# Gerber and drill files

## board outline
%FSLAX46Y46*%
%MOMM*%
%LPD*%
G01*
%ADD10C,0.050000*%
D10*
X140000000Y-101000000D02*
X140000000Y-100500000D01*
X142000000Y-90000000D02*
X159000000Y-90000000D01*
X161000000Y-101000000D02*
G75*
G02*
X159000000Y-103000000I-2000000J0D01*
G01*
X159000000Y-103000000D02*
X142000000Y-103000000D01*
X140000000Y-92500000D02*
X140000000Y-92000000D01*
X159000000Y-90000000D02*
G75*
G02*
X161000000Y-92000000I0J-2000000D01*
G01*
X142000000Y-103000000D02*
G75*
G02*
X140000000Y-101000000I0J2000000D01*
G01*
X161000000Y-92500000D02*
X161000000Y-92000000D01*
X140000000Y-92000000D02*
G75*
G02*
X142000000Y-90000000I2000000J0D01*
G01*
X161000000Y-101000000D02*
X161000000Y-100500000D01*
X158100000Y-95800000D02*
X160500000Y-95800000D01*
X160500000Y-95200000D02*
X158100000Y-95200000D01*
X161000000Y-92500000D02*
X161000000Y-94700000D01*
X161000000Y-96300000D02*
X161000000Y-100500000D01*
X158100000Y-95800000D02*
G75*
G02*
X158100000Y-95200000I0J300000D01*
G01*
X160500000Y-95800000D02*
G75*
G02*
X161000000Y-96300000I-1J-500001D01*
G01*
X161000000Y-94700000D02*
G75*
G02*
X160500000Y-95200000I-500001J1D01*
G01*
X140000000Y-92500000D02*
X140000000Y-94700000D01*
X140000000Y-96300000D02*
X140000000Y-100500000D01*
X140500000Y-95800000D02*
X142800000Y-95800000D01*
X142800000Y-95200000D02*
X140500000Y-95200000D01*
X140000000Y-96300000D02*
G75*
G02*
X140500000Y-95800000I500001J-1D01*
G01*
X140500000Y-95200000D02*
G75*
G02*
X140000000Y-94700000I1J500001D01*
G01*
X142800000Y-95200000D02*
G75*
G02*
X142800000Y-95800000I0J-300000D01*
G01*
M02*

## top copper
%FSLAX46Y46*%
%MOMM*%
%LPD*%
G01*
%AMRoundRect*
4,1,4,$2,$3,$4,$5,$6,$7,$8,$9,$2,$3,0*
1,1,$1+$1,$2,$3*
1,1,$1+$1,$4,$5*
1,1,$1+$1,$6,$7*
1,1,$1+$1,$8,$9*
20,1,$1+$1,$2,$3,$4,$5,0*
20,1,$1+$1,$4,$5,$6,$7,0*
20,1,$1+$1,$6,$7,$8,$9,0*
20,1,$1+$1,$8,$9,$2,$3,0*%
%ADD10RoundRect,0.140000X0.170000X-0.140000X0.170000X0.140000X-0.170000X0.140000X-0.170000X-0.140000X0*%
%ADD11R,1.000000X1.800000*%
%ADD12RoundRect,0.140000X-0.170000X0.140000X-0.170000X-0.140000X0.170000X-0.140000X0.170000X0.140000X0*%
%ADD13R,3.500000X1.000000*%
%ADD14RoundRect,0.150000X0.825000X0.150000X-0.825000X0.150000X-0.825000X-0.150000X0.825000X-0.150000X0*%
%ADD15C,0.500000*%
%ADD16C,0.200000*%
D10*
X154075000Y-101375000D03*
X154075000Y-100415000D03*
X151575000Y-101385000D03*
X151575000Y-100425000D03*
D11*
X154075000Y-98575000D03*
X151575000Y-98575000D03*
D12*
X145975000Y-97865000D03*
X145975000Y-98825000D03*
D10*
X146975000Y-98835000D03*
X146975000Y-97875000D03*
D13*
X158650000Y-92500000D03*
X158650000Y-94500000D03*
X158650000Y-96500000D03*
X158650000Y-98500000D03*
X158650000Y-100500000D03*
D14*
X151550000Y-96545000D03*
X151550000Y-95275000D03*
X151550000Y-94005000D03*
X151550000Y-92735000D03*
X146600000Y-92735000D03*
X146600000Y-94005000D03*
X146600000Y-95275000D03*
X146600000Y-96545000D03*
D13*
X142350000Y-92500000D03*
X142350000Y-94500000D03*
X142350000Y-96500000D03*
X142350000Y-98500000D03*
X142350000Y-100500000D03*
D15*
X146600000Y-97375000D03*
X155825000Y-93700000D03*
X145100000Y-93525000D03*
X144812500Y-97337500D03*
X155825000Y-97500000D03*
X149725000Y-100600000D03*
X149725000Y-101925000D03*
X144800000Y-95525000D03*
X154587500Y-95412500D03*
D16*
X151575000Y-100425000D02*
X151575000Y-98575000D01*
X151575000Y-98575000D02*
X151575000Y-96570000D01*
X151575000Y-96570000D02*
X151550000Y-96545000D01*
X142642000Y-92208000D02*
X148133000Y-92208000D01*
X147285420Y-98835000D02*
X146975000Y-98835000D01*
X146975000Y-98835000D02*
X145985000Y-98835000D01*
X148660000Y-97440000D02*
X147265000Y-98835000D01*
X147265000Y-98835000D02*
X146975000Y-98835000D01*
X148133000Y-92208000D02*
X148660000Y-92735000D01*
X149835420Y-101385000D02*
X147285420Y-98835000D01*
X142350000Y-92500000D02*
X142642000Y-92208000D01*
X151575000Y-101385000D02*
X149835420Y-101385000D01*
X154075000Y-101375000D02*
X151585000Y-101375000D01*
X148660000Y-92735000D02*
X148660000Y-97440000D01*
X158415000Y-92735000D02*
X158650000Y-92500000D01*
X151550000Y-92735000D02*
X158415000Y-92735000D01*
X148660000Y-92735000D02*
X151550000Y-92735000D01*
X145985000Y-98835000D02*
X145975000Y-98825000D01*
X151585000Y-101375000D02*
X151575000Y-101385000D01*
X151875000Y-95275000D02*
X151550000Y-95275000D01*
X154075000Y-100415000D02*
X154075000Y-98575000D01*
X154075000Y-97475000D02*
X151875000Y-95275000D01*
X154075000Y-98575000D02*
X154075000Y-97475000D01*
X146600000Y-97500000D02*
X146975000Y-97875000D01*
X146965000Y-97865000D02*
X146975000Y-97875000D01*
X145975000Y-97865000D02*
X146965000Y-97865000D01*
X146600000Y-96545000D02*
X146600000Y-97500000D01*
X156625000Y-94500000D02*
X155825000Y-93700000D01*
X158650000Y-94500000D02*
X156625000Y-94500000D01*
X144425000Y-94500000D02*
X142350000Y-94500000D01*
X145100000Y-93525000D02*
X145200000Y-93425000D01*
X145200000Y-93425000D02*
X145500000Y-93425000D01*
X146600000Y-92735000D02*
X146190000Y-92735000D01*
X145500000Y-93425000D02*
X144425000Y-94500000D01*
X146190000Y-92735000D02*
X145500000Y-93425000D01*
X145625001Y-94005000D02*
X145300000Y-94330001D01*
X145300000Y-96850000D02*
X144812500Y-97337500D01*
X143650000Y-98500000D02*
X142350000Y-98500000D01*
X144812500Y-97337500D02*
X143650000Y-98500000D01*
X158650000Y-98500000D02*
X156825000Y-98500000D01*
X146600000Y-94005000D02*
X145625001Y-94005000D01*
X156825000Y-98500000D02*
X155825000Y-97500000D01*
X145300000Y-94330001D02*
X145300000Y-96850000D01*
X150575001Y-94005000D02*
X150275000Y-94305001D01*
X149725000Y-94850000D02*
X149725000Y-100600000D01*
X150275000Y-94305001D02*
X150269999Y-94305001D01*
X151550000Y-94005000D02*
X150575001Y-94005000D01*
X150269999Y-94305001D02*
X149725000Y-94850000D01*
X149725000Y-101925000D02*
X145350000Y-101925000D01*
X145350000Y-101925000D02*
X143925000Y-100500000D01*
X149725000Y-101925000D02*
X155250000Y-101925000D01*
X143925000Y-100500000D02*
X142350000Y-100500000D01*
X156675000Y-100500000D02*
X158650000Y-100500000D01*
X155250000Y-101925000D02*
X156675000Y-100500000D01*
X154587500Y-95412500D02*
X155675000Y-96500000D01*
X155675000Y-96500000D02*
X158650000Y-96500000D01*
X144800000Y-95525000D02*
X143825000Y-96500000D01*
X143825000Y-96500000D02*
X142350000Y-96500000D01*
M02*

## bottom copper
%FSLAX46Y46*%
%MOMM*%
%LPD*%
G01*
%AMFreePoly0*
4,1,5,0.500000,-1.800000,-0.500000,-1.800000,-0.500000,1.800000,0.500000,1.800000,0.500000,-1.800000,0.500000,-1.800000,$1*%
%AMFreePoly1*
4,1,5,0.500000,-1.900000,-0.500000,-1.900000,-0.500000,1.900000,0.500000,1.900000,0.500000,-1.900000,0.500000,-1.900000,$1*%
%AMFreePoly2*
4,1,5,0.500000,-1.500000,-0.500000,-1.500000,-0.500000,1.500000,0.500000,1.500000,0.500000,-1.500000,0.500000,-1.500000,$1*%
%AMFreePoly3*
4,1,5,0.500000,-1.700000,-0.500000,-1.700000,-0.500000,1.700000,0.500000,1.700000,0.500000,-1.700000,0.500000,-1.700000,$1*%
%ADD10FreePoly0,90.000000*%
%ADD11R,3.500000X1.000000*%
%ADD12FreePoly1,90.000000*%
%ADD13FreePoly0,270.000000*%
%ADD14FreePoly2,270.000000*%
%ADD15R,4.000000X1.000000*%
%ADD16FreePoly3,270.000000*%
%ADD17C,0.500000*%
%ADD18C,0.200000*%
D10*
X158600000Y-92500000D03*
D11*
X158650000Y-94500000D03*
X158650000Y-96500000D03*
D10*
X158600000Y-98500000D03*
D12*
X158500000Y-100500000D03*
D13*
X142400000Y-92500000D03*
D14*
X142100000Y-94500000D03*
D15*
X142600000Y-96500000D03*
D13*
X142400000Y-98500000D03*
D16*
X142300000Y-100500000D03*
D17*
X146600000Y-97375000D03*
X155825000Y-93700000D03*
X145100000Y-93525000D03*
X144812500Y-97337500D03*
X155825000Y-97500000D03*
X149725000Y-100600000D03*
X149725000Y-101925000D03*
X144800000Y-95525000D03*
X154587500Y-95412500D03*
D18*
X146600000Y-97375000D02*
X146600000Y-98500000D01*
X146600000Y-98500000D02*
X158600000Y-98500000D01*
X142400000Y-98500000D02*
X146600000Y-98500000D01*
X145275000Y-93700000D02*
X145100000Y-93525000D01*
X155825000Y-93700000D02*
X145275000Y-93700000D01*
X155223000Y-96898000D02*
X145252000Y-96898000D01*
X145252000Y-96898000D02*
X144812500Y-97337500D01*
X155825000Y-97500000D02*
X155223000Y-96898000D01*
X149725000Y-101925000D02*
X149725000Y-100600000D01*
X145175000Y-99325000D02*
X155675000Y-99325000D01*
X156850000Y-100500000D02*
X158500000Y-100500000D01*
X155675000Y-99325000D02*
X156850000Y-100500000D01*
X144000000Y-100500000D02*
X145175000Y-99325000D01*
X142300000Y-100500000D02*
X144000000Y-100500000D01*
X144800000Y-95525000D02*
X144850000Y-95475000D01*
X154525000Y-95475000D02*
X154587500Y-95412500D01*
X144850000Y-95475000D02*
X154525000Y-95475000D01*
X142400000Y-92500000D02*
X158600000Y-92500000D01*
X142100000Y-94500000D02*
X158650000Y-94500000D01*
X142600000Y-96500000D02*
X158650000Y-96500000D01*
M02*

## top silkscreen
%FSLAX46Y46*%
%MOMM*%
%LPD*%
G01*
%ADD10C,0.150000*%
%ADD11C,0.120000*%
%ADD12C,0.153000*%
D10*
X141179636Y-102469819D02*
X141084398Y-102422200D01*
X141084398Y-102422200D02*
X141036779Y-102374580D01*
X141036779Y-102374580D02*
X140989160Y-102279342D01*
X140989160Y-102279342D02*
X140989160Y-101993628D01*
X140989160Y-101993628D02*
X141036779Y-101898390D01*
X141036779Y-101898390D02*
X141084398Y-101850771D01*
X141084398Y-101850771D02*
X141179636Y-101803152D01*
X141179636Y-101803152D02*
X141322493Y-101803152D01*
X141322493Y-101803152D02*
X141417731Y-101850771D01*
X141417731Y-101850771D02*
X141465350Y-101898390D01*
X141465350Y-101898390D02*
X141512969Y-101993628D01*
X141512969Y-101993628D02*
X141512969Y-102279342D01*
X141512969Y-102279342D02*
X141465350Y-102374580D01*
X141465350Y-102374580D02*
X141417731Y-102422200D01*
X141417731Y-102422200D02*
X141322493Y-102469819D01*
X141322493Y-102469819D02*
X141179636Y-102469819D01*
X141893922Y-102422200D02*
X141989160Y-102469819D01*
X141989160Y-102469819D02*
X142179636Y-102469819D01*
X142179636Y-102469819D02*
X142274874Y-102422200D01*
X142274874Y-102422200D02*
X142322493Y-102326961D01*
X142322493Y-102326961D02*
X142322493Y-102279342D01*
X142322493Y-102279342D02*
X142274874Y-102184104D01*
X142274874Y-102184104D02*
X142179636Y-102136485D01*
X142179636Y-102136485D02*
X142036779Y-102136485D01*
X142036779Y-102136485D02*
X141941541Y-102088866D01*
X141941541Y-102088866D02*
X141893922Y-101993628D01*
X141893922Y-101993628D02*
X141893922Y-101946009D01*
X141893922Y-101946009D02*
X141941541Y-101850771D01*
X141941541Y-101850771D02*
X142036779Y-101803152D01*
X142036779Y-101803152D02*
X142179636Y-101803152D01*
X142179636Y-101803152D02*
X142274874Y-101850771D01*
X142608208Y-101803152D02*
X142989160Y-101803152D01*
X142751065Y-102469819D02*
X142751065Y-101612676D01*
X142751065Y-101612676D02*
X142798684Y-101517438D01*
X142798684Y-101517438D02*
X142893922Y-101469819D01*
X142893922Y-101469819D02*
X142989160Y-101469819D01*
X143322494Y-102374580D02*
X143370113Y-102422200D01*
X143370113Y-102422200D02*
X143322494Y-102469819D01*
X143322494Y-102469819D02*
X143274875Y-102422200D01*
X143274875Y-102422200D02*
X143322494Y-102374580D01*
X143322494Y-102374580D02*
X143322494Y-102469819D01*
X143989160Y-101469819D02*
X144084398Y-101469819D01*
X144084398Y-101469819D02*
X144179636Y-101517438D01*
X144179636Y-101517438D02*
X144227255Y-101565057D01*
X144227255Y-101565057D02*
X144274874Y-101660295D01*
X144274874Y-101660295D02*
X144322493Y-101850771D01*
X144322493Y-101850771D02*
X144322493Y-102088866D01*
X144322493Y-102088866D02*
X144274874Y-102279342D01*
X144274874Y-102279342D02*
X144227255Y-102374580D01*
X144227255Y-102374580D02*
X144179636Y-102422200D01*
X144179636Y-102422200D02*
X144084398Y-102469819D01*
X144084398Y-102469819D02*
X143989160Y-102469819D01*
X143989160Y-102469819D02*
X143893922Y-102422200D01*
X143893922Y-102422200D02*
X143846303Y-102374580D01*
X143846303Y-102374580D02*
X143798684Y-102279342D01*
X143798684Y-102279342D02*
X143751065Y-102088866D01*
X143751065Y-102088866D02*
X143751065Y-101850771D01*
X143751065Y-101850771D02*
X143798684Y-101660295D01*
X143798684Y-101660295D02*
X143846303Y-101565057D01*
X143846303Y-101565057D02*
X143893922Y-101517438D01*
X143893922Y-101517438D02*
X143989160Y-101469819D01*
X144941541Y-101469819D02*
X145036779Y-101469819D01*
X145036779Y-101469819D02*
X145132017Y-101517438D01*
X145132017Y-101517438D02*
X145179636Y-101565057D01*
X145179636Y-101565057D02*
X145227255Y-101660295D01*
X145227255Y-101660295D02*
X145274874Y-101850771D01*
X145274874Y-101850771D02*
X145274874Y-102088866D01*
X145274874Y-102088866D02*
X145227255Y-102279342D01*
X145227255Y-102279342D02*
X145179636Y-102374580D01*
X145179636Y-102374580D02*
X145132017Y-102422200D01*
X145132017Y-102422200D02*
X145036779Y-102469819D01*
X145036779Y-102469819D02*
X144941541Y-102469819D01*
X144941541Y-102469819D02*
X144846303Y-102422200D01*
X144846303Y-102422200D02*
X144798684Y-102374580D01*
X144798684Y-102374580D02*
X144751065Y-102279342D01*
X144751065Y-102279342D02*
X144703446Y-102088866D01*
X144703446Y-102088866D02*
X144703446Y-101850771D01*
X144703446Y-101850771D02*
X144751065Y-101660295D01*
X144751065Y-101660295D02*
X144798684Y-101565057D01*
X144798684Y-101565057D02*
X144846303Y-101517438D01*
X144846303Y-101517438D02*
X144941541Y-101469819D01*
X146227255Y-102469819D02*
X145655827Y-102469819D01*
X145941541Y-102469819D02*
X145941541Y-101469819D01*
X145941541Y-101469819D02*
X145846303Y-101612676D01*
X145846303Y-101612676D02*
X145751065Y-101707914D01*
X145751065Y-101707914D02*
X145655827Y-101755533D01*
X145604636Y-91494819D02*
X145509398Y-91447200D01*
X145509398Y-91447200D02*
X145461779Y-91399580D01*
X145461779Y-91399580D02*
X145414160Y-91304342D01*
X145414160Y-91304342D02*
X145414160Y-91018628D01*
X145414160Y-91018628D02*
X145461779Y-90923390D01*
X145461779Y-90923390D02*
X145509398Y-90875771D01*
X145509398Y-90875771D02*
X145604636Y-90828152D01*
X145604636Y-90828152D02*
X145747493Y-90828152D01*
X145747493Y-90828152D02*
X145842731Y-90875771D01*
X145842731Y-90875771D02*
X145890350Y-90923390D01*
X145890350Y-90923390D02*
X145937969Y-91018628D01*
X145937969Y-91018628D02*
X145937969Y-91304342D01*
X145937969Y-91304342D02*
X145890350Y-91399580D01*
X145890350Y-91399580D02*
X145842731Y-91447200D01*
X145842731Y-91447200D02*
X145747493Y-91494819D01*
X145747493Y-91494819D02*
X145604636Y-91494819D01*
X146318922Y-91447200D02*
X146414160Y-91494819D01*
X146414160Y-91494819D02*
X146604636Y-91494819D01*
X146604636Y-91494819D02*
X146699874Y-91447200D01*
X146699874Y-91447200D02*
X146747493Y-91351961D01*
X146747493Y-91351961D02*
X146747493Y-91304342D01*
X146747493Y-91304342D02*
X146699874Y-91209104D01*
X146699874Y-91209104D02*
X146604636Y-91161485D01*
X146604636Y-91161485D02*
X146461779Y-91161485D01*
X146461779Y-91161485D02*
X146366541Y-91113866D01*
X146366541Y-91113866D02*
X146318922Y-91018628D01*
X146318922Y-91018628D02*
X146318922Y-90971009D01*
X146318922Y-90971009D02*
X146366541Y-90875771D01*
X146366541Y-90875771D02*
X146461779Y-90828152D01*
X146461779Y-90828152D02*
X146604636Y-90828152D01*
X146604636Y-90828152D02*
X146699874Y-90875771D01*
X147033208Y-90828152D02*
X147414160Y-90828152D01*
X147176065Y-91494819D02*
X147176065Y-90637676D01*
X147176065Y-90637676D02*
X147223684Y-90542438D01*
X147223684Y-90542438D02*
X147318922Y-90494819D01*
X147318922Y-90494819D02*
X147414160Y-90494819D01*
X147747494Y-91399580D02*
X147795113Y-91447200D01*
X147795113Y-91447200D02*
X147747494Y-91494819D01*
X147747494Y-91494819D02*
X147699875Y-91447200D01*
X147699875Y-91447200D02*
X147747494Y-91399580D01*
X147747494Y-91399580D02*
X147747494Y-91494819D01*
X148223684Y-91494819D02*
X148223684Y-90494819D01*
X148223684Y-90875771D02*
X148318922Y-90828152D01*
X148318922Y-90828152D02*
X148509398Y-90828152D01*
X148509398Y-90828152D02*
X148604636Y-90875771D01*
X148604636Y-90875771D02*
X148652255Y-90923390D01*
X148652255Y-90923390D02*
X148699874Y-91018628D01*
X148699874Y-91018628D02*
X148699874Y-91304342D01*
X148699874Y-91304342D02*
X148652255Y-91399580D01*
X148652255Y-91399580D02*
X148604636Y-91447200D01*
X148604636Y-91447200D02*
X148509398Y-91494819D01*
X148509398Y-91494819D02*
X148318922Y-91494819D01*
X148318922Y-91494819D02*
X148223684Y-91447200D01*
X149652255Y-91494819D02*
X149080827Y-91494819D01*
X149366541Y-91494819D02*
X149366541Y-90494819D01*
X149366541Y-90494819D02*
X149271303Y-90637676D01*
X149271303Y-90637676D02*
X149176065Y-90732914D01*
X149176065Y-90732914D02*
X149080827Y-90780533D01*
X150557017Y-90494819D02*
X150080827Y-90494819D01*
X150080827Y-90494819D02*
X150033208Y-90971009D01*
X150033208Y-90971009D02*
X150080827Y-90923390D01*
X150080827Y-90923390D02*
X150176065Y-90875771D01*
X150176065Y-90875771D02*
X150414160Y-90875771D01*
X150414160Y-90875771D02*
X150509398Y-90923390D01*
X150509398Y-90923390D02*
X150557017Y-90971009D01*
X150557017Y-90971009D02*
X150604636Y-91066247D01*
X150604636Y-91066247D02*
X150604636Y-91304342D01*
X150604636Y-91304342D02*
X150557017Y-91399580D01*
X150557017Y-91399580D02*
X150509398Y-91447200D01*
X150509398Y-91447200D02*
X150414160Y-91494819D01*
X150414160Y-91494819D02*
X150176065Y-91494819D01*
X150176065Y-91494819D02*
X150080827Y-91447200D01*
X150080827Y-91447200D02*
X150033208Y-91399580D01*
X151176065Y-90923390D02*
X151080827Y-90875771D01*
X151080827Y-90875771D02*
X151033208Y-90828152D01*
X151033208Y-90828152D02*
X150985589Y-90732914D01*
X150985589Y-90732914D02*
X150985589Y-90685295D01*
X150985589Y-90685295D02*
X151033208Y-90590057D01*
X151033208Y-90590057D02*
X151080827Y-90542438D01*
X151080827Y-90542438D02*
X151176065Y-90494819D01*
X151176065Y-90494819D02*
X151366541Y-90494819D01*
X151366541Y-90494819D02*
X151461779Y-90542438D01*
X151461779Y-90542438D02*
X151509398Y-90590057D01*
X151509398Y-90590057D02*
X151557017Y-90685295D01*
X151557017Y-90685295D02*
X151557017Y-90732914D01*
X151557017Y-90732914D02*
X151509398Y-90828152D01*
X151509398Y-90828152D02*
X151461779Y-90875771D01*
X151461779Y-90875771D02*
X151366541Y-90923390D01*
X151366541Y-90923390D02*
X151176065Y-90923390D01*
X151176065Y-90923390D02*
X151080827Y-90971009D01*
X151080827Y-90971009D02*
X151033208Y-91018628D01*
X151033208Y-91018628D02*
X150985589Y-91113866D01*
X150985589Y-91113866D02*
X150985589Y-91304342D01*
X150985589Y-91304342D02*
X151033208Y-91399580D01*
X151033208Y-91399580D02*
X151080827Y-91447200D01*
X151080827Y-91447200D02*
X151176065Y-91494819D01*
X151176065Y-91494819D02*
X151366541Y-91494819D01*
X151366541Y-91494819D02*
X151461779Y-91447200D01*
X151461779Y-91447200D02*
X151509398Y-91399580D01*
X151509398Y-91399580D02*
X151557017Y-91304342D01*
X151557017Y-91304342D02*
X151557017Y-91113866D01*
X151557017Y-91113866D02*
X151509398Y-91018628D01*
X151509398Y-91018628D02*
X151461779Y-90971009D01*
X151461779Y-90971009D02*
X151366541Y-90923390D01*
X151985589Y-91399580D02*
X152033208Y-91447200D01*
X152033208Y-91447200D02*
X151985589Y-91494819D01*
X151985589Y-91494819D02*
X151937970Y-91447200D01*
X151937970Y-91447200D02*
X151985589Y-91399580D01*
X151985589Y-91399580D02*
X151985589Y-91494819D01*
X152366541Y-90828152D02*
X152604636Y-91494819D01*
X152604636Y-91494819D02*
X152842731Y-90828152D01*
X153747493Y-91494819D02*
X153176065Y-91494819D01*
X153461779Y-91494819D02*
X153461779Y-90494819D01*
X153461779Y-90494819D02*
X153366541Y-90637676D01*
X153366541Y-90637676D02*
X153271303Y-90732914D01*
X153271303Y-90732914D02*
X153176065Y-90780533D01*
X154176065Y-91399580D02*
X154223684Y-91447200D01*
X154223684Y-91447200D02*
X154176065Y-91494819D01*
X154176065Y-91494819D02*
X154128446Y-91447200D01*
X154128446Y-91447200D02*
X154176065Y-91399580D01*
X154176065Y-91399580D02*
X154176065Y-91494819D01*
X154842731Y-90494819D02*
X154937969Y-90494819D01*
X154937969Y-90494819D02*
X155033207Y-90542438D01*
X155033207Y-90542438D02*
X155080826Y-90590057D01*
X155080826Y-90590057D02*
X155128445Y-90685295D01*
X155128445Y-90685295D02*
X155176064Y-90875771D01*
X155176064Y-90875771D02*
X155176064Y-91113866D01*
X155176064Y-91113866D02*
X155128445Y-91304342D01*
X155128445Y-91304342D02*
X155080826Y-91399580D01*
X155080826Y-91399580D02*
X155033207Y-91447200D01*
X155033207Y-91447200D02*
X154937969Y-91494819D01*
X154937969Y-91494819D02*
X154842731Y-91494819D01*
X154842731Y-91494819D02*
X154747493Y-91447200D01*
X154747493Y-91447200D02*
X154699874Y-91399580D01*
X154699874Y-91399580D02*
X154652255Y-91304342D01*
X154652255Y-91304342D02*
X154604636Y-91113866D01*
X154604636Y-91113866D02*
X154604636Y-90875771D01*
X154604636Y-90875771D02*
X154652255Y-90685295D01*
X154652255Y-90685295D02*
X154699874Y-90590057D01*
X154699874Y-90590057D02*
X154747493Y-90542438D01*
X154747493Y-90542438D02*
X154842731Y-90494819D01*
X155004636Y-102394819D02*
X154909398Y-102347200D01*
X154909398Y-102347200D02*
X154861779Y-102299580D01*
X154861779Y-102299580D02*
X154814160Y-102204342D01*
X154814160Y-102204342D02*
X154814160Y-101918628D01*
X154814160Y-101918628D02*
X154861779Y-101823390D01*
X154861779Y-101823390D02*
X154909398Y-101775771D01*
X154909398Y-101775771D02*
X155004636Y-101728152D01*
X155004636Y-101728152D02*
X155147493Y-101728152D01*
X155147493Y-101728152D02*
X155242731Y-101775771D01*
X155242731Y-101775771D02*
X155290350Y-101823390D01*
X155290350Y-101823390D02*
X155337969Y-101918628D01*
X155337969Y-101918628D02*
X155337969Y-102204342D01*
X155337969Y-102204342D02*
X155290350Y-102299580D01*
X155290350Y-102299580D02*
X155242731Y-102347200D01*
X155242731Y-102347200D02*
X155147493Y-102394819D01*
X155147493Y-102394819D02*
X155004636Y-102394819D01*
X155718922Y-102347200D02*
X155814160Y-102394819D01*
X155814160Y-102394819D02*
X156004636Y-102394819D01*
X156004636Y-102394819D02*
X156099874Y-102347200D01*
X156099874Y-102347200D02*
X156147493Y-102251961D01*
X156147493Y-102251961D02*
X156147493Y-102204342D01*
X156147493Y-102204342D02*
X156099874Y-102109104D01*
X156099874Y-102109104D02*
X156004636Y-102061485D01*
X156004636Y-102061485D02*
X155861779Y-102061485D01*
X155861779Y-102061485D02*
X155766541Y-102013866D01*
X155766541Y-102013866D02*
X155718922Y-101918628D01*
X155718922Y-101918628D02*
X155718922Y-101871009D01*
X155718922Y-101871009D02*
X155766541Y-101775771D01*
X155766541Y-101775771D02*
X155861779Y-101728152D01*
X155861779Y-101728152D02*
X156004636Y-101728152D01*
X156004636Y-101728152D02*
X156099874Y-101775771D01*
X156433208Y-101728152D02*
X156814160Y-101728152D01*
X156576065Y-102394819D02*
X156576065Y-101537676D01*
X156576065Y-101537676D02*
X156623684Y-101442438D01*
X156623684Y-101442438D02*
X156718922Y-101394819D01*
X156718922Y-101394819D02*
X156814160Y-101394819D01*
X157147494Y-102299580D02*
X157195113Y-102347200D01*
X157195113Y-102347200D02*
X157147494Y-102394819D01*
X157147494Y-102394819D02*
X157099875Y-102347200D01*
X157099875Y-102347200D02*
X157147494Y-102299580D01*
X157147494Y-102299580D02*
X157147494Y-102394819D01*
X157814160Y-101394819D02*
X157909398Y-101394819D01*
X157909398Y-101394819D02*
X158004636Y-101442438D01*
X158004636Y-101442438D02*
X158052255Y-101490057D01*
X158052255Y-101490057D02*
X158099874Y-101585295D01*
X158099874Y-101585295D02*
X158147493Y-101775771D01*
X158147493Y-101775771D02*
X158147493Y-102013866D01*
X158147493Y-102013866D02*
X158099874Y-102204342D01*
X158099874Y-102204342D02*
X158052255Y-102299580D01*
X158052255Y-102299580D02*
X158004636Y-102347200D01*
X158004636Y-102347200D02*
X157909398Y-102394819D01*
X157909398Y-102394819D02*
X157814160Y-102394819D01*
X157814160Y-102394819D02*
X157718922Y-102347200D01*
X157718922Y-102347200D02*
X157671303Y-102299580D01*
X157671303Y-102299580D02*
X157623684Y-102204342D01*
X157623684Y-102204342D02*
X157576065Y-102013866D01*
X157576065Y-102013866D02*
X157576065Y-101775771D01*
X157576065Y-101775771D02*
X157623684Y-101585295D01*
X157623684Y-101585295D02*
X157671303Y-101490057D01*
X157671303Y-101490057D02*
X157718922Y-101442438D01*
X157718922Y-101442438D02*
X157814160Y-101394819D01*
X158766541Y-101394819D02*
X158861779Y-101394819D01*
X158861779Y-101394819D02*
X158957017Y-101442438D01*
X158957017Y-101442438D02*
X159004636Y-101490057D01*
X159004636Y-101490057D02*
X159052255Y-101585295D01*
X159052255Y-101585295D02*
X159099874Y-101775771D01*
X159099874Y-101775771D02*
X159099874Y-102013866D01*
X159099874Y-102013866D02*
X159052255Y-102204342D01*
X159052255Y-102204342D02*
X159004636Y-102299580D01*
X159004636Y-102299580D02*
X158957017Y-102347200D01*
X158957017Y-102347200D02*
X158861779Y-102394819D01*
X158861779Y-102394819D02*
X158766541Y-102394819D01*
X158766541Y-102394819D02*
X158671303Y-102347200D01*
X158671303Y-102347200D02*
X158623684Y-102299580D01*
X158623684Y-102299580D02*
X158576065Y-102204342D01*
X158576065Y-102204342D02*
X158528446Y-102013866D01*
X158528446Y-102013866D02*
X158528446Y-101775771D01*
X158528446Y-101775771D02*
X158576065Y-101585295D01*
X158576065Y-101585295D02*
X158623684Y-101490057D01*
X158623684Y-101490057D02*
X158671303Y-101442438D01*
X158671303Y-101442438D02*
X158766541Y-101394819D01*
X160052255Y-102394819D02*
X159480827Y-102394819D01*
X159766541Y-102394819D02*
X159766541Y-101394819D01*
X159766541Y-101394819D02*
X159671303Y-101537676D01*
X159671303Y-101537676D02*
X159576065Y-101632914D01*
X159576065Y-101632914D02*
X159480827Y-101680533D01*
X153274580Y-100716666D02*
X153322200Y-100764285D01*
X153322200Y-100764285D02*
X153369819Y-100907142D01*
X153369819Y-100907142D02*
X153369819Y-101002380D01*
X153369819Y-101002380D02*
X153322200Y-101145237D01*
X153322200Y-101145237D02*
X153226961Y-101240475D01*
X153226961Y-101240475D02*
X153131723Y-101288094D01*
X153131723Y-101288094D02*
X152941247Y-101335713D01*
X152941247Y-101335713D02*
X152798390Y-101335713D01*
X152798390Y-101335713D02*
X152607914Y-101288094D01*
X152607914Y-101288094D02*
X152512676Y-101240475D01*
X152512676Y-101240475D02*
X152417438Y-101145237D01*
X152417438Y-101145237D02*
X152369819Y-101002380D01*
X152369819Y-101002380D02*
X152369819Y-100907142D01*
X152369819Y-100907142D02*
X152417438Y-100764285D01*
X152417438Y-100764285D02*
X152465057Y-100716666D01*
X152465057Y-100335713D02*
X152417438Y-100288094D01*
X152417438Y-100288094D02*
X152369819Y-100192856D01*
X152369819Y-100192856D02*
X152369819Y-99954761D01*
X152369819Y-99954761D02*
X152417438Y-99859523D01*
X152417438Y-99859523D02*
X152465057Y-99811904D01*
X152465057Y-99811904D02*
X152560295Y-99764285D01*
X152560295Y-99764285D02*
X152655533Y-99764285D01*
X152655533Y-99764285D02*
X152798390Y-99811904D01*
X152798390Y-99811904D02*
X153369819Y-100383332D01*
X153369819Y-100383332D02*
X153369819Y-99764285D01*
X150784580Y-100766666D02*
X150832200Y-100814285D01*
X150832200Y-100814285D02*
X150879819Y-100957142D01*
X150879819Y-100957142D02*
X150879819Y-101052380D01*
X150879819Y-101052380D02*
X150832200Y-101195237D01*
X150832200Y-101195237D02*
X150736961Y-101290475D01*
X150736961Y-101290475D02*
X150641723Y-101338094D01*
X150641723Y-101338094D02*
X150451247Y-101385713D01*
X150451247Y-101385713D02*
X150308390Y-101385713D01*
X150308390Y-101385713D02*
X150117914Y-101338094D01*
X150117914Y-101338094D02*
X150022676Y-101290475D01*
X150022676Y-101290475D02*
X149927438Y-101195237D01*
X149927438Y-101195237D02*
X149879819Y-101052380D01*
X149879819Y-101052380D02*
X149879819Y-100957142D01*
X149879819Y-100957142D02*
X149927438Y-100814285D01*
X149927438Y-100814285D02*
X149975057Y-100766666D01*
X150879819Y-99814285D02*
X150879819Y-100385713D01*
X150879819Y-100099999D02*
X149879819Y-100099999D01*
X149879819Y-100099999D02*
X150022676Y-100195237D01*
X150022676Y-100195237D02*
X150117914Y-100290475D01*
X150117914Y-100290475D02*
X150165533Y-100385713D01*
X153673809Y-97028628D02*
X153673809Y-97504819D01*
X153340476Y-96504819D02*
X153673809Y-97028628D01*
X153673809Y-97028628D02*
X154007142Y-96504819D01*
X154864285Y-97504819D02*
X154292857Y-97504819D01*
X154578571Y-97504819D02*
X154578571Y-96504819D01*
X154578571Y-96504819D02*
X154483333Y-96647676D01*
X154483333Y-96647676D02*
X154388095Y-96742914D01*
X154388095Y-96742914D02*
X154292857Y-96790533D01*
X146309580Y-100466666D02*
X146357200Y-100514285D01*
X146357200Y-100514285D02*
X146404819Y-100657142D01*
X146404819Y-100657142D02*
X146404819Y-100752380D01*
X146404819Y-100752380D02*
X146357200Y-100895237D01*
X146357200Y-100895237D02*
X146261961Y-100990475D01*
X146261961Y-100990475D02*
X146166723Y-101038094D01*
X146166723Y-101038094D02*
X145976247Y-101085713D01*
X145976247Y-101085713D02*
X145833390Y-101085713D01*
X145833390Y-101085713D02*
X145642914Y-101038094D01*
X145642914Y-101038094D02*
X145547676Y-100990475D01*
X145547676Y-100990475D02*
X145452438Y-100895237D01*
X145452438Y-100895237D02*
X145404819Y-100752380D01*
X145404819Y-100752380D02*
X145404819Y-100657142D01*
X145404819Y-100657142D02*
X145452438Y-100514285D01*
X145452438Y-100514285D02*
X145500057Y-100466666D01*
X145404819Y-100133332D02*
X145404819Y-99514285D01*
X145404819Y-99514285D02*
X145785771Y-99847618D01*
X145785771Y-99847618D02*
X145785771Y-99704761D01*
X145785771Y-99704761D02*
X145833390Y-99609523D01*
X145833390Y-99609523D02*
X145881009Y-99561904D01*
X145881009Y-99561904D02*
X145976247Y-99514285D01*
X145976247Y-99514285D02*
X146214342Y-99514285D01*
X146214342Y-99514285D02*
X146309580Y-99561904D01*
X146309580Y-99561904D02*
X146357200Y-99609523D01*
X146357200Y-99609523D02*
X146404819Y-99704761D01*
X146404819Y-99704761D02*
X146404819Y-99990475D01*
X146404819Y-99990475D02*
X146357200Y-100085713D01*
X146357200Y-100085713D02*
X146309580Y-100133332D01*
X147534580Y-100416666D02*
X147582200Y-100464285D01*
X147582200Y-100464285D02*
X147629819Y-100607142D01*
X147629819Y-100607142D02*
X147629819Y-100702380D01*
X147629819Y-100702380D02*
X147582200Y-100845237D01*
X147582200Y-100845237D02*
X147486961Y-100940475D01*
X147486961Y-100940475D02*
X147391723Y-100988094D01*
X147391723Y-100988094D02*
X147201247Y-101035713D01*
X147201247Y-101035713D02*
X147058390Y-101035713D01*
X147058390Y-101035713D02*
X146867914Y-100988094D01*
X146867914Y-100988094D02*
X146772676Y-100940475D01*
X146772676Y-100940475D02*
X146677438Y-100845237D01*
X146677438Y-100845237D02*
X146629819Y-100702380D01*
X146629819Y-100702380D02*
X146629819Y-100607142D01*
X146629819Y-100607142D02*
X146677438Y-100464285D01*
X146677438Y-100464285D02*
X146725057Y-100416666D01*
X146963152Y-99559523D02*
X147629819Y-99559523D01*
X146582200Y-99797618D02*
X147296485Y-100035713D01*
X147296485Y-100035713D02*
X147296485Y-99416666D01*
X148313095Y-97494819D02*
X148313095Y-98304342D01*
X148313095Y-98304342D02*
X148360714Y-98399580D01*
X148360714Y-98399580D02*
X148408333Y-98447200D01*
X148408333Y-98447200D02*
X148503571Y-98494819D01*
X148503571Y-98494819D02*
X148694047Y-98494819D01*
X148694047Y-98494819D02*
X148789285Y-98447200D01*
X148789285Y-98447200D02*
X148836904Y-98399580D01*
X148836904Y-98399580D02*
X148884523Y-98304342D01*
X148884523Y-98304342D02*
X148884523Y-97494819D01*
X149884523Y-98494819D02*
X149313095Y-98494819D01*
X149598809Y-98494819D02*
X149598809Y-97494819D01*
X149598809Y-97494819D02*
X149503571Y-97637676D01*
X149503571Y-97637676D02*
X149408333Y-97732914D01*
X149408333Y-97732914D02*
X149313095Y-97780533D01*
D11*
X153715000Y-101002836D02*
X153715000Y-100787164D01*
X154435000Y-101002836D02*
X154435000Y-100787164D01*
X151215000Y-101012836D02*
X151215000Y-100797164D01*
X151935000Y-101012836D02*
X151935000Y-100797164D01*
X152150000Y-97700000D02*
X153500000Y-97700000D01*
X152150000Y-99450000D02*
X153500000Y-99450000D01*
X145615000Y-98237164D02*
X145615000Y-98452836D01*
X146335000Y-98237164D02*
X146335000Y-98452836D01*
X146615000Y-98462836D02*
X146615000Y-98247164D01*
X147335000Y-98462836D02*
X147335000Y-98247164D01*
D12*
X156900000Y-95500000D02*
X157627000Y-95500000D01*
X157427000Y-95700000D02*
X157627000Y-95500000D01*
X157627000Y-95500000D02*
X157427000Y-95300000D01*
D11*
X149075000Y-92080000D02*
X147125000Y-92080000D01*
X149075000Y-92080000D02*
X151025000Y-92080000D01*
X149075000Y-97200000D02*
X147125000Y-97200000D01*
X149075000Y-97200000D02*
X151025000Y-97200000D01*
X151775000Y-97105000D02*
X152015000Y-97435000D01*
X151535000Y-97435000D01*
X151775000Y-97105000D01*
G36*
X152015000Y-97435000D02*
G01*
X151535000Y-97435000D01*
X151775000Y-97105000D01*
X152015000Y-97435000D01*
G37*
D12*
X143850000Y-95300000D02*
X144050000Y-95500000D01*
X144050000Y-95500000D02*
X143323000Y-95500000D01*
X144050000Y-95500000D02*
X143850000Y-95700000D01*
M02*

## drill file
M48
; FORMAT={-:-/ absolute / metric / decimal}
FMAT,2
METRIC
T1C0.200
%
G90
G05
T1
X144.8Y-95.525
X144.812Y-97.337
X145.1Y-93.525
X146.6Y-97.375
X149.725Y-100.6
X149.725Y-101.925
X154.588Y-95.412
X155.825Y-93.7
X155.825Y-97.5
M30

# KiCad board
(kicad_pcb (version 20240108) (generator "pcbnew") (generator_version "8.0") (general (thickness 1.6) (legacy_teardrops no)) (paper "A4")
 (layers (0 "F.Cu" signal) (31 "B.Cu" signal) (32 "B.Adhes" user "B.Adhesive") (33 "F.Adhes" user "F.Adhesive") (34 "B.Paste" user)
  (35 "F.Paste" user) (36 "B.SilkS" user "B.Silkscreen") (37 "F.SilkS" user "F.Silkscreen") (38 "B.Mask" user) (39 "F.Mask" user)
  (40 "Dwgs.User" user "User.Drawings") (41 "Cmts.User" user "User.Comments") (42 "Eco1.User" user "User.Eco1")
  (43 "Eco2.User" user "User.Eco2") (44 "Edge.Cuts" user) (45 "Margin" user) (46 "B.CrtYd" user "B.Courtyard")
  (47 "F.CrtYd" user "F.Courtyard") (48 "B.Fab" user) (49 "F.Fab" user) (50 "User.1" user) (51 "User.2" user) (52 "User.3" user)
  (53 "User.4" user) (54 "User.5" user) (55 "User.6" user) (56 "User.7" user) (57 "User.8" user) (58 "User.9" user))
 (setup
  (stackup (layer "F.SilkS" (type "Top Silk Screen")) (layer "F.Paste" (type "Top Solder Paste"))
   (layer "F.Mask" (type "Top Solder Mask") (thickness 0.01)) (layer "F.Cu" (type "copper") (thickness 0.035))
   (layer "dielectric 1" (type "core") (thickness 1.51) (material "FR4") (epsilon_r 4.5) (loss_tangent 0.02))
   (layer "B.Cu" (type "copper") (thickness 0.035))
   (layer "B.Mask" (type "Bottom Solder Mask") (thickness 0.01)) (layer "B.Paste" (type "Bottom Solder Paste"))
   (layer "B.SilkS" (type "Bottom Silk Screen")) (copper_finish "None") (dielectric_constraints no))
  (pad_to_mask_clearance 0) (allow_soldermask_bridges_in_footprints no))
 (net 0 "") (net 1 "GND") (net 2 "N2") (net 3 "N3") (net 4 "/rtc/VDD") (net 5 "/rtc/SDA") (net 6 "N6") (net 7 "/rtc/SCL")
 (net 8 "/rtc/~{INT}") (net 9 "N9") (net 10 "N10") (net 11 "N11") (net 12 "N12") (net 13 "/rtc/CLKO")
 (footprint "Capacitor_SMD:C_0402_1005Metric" (layer "F.Cu") (at 154.075 100.895 90)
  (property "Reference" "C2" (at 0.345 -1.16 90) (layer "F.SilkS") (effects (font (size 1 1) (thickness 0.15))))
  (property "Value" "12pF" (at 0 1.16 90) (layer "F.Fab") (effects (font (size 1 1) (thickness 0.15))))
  (fp_line (start -0.107836 -0.36) (end 0.107836 -0.36) (stroke (width 0.12) (type solid)) (layer "F.SilkS"))
  (fp_line (start -0.107836 0.36) (end 0.107836 0.36) (stroke (width 0.12) (type solid)) (layer "F.SilkS"))
  (pad "1" smd roundrect (at -0.48 0 90) (size 0.56 0.62) (layers "F.Cu" "F.Paste" "F.Mask") (roundrect_rratio 0.25) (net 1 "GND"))
  (pad "2" smd roundrect (at 0.48 0 90) (size 0.56 0.62) (layers "F.Cu" "F.Paste" "F.Mask") (roundrect_rratio 0.25) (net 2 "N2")))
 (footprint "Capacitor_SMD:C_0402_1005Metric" (layer "F.Cu") (at 151.575 100.905 90)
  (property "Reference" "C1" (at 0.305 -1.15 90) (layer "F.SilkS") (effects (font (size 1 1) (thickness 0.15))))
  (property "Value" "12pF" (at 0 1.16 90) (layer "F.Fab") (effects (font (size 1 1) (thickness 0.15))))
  (fp_line (start -0.107836 -0.36) (end 0.107836 -0.36) (stroke (width 0.12) (type solid)) (layer "F.SilkS"))
  (fp_line (start -0.107836 0.36) (end 0.107836 0.36) (stroke (width 0.12) (type solid)) (layer "F.SilkS"))
  (pad "1" smd roundrect (at -0.48 0 90) (size 0.56 0.62) (layers "F.Cu" "F.Paste" "F.Mask") (roundrect_rratio 0.25) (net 1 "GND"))
  (pad "2" smd roundrect (at 0.48 0 90) (size 0.56 0.62) (layers "F.Cu" "F.Paste" "F.Mask") (roundrect_rratio 0.25) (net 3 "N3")))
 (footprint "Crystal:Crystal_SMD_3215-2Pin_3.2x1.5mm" (layer "F.Cu") (at 152.825 98.575)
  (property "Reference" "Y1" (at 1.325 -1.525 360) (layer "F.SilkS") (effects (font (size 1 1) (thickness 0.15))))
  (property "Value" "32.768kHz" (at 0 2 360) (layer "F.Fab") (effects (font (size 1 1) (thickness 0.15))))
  (fp_line (start -0.675 -0.875) (end 0.675 -0.875) (stroke (width 0.12) (type solid)) (layer "F.SilkS"))
  (fp_line (start -0.675 0.875) (end 0.675 0.875) (stroke (width 0.12) (type solid)) (layer "F.SilkS"))
  (pad "1" smd rect (at 1.25 0) (size 1 1.8) (layers "F.Cu" "F.Paste" "F.Mask") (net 2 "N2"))
  (pad "2" smd rect (at -1.25 0) (size 1 1.8) (layers "F.Cu" "F.Paste" "F.Mask") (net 3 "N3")))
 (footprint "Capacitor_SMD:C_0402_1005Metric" (layer "F.Cu") (at 145.975 98.345 -90)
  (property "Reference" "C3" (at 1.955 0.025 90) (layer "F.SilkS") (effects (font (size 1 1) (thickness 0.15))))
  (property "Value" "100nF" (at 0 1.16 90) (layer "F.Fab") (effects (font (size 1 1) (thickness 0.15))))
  (fp_line (start -0.107836 0.36) (end 0.107836 0.36) (stroke (width 0.12) (type solid)) (layer "F.SilkS"))
  (fp_line (start -0.107836 -0.36) (end 0.107836 -0.36) (stroke (width 0.12) (type solid)) (layer "F.SilkS"))
  (pad "1" smd roundrect (at -0.48 0 270) (size 0.56 0.62) (layers "F.Cu" "F.Paste" "F.Mask") (roundrect_rratio 0.25) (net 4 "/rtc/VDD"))
  (pad "2" smd roundrect (at 0.48 0 270) (size 0.56 0.62) (layers "F.Cu" "F.Paste" "F.Mask") (roundrect_rratio 0.25) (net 1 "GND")))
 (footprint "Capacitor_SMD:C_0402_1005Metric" (layer "F.Cu") (at 146.975 98.355 90)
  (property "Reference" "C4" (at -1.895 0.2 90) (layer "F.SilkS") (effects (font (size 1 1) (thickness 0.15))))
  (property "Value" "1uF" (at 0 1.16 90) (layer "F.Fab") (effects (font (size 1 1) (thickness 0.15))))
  (fp_line (start -0.107836 -0.36) (end 0.107836 -0.36) (stroke (width 0.12) (type solid)) (layer "F.SilkS"))
  (fp_line (start -0.107836 0.36) (end 0.107836 0.36) (stroke (width 0.12) (type solid)) (layer "F.SilkS"))
  (pad "1" smd roundrect (at -0.48 0 90) (size 0.56 0.62) (layers "F.Cu" "F.Paste" "F.Mask") (roundrect_rratio 0.25) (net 1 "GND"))
  (pad "2" smd roundrect (at 0.48 0 90) (size 0.56 0.62) (layers "F.Cu" "F.Paste" "F.Mask") (roundrect_rratio 0.25) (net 4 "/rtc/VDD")))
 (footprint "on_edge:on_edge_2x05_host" (layer "F.Cu") (at 161 96.5 -90)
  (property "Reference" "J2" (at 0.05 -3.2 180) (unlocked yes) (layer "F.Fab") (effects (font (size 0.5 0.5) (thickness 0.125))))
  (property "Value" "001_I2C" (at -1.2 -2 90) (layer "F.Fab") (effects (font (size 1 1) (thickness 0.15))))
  (fp_line (start -1 4.1) (end -1 3.373) (stroke (width 0.153) (type solid)) (layer "F.SilkS"))
  (fp_line (start -0.8 3.573) (end -1 3.373) (stroke (width 0.153) (type solid)) (layer "F.SilkS"))
  (fp_line (start -1 3.373) (end -1.2 3.573) (stroke (width 0.153) (type solid)) (layer "F.SilkS"))
  (fp_line (start -0.7 2.9) (end -0.7 0.5) (stroke (width 0.05) (type solid)) (layer "Edge.Cuts"))
  (fp_line (start -1.3 0.5) (end -1.3 2.9) (stroke (width 0.05) (type solid)) (layer "Edge.Cuts"))
  (fp_line (start -4 0) (end -1.8 0) (stroke (width 0.05) (type solid)) (layer "Edge.Cuts"))
  (fp_line (start -0.2 0) (end 4 0) (stroke (width 0.05) (type solid)) (layer "Edge.Cuts"))
  (fp_arc (start -0.7 2.9) (mid -1 3.2) (end -1.3 2.9) (stroke (width 0.05) (type solid)) (layer "Edge.Cuts"))
  (fp_arc (start -0.7 0.5) (mid -0.553553 0.146447) (end -0.2 0) (stroke (width 0.05) (type solid)) (layer "Edge.Cuts"))
  (fp_arc (start -1.8 0) (mid -1.446447 0.146447) (end -1.3 0.5) (stroke (width 0.05) (type solid)) (layer "Edge.Cuts"))
  (pad "1" smd rect (at -4 2.35 270) (size 1 3.5) (layers "F.Cu" "F.Mask") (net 1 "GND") (zone_connect 0))
  (pad "2" smd rect (at -2 2.35 270) (size 1 3.5) (layers "F.Cu" "F.Mask") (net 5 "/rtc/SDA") (zone_connect 0))
  (pad "3" smd rect (at 0 2.35 270) (size 1 3.5) (layers "F.Cu" "F.Mask") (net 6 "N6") (zone_connect 0))
  (pad "4" smd rect (at 2 2.35 270) (size 1 3.5) (layers "F.Cu" "F.Mask") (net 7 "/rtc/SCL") (zone_connect 0))
  (pad "5" smd rect (at 4 2.35 270) (size 1 3.5) (layers "F.Cu" "F.Mask") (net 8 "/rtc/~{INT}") (zone_connect 0))
  (pad "6" smd custom (at -4 2.4 90) (size 1 3.6) (layers "B.Cu" "B.Mask") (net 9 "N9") (zone_connect 0)
   (options (clearance outline) (anchor rect)) (primitives))
  (pad "7" smd rect (at -2 2.35 90) (size 1 3.5) (layers "B.Cu" "B.Mask") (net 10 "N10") (zone_connect 0))
  (pad "8" smd rect (at 0 2.35 90) (size 1 3.5) (layers "B.Cu" "B.Mask") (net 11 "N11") (zone_connect 0))
  (pad "9" smd custom (at 2 2.4 90) (size 1 3.6) (layers "B.Cu" "B.Mask") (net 4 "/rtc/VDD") (zone_connect 0)
   (options (clearance outline) (anchor rect)) (primitives))
  (pad "10" smd custom (at 4 2.5 90) (size 1 3.8) (layers "B.Cu" "B.Mask") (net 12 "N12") (zone_connect 0)
   (options (clearance outline) (anchor rect)) (primitives))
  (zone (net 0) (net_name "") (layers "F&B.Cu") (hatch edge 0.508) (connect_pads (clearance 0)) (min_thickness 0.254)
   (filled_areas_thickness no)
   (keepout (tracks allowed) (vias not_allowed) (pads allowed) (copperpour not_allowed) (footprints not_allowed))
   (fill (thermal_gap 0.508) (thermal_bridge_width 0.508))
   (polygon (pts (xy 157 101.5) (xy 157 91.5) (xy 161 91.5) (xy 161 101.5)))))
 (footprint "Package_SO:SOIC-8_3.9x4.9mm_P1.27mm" (layer "F.Cu") (at 149.075 94.64 180)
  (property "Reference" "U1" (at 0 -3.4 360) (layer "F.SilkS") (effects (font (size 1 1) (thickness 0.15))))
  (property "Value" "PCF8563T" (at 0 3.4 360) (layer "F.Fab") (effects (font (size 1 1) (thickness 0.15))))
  (fp_line (start 0 2.56) (end 1.95 2.56) (stroke (width 0.12) (type solid)) (layer "F.SilkS"))
  (fp_line (start 0 2.56) (end -1.95 2.56) (stroke (width 0.12) (type solid)) (layer "F.SilkS"))
  (fp_line (start 0 -2.56) (end 1.95 -2.56) (stroke (width 0.12) (type solid)) (layer "F.SilkS"))
  (fp_line (start 0 -2.56) (end -1.95 -2.56) (stroke (width 0.12) (type solid)) (layer "F.SilkS"))
  (fp_poly
   (pts (xy -2.7 -2.465) (xy -2.94 -2.795) (xy -2.46 -2.795) (xy -2.7 -2.465)) (stroke (width 0.12) (type solid)) (fill solid)
   (layer "F.SilkS"))
  (pad "1" smd roundrect (at -2.475 -1.905 180) (size 1.95 0.6) (layers "F.Cu" "F.Paste" "F.Mask") (roundrect_rratio 0.25) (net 3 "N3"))
  (pad "2" smd roundrect (at -2.475 -0.635 180) (size 1.95 0.6) (layers "F.Cu" "F.Paste" "F.Mask") (roundrect_rratio 0.25) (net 2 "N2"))
  (pad "3" smd roundrect (at -2.475 0.635 180) (size 1.95 0.6) (layers "F.Cu" "F.Paste" "F.Mask") (roundrect_rratio 0.25)
   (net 8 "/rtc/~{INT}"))
  (pad "4" smd roundrect (at -2.475 1.905 180) (size 1.95 0.6) (layers "F.Cu" "F.Paste" "F.Mask") (roundrect_rratio 0.25) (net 1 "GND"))
  (pad "5" smd roundrect (at 2.475 1.905 180) (size 1.95 0.6) (layers "F.Cu" "F.Paste" "F.Mask") (roundrect_rratio 0.25) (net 5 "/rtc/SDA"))
  (pad "6" smd roundrect (at 2.475 0.635 180) (size 1.95 0.6) (layers "F.Cu" "F.Paste" "F.Mask") (roundrect_rratio 0.25) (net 7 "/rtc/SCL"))
  (pad "7" smd roundrect (at 2.475 -0.635 180) (size 1.95 0.6) (layers "F.Cu" "F.Paste" "F.Mask") (roundrect_rratio 0.25)
   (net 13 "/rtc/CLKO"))
  (pad "8" smd roundrect (at 2.475 -1.905 180) (size 1.95 0.6) (layers "F.Cu" "F.Paste" "F.Mask") (roundrect_rratio 0.25) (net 4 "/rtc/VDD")))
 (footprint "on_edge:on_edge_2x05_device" (layer "F.Cu") (at 140 96.5 -90)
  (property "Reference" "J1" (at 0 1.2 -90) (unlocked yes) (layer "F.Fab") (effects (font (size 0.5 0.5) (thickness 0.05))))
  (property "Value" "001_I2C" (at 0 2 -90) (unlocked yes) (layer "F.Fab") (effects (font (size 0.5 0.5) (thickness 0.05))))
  (fp_line (start -1.2 -3.85) (end -1 -4.05) (stroke (width 0.153) (type solid)) (layer "F.SilkS"))
  (fp_line (start -1 -4.05) (end -1 -3.323) (stroke (width 0.153) (type solid)) (layer "F.SilkS"))
  (fp_line (start -1 -4.05) (end -0.8 -3.85) (stroke (width 0.153) (type solid)) (layer "F.SilkS"))
  (fp_line (start -4 0) (end -1.8 0) (stroke (width 0.05) (type solid)) (layer "Edge.Cuts"))
  (fp_line (start -0.2 0) (end 4 0) (stroke (width 0.05) (type solid)) (layer "Edge.Cuts"))
  (fp_line (start -0.7 -0.5) (end -0.7 -2.8) (stroke (width 0.05) (type solid)) (layer "Edge.Cuts"))
  (fp_line (start -1.3 -2.8) (end -1.3 -0.5) (stroke (width 0.05) (type solid)) (layer "Edge.Cuts"))
  (fp_arc (start -0.2 0) (mid -0.553553 -0.146447) (end -0.7 -0.5) (stroke (width 0.05) (type solid)) (layer "Edge.Cuts"))
  (fp_arc (start -1.3 -0.5) (mid -1.446447 -0.146447) (end -1.8 0) (stroke (width 0.05) (type solid)) (layer "Edge.Cuts"))
  (fp_arc (start -1.3 -2.8) (mid -1 -3.1) (end -0.7 -2.8) (stroke (width 0.05) (type solid)) (layer "Edge.Cuts"))
  (pad "1" smd rect (at -4 -2.35 90) (size 1 3.5) (layers "F.Cu" "F.Mask") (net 1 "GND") (zone_connect 0))
  (pad "2" smd rect (at -2 -2.35 270) (size 1 3.5) (layers "F.Cu" "F.Mask") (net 5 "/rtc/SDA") (zone_connect 0))
  (pad "3" smd rect (at 0 -2.35 270) (size 1 3.5) (layers "F.Cu" "F.Mask") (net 6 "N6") (zone_connect 0))
  (pad "4" smd rect (at 2 -2.35 90) (size 1 3.5) (layers "F.Cu" "F.Mask") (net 7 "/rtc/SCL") (zone_connect 0))
  (pad "5" smd rect (at 4 -2.35 90) (size 1 3.5) (layers "F.Cu" "F.Mask") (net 8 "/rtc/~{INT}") (zone_connect 0))
  (pad "6" smd custom (at -4 -2.4 270) (size 1 3.6) (layers "B.Cu" "B.Mask") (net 9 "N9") (zone_connect 0)
   (options (clearance outline) (anchor rect)) (primitives))
  (pad "7" smd custom (at -2 -2.1 270) (size 1 3) (layers "B.Cu" "B.Mask") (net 10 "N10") (zone_connect 0)
   (options (clearance outline) (anchor rect)) (primitives))
  (pad "8" smd rect (at 0 -2.6 270) (size 1 4) (layers "B.Cu" "B.Mask") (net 11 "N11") (zone_connect 0))
  (pad "9" smd custom (at 2 -2.4 270) (size 1 3.6) (layers "B.Cu" "B.Mask") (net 4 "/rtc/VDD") (zone_connect 0)
   (options (clearance outline) (anchor rect)) (primitives))
  (pad "10" smd custom (at 4 -2.3 270) (size 1 3.4) (layers "B.Cu" "B.Mask") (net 12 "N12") (zone_connect 0)
   (options (clearance outline) (anchor rect)) (primitives))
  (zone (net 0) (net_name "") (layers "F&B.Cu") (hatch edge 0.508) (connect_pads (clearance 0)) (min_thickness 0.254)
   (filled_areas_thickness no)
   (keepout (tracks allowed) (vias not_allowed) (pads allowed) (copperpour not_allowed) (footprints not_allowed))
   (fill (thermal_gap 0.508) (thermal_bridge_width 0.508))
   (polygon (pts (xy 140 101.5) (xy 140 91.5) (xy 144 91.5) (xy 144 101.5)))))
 (gr_line (start 140 101) (end 140 100.5) (stroke (width 0.05) (type solid)) (layer "Edge.Cuts"))
 (gr_line (start 142 90) (end 159 90) (stroke (width 0.05) (type solid)) (layer "Edge.Cuts"))
 (gr_arc (start 161 101) (mid 160.414214 102.414214) (end 159 103) (stroke (width 0.05) (type solid)) (layer "Edge.Cuts"))
 (gr_line (start 159 103) (end 142 103) (stroke (width 0.05) (type solid)) (layer "Edge.Cuts"))
 (gr_line (start 140 92.5) (end 140 92) (stroke (width 0.05) (type solid)) (layer "Edge.Cuts"))
 (gr_arc (start 159 90) (mid 160.414214 90.585786) (end 161 92) (stroke (width 0.05) (type solid)) (layer "Edge.Cuts"))
 (gr_arc (start 142 103) (mid 140.585786 102.414214) (end 140 101) (stroke (width 0.05) (type solid)) (layer "Edge.Cuts"))
 (gr_line (start 161 92.5) (end 161 92) (stroke (width 0.05) (type solid)) (layer "Edge.Cuts"))
 (gr_arc (start 140 92) (mid 140.585786 90.585786) (end 142 90) (stroke (width 0.05) (type solid)) (layer "Edge.Cuts"))
 (gr_line (start 161 101) (end 161 100.5) (stroke (width 0.05) (type solid)) (layer "Edge.Cuts"))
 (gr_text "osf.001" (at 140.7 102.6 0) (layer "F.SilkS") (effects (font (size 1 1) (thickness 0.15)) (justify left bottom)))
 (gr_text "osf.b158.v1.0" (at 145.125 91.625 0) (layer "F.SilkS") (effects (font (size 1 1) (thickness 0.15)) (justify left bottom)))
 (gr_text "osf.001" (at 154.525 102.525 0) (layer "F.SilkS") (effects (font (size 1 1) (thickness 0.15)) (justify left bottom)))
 (segment (start 151.575 100.425) (end 151.575 98.575) (width 0.2) (layer "F.Cu") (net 3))
 (segment (start 151.575 98.575) (end 151.575 96.57) (width 0.2) (layer "F.Cu") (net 3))
 (segment (start 151.575 96.57) (end 151.55 96.545) (width 0.2) (layer "F.Cu") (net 3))
 (segment (start 142.642 92.208) (end 148.133 92.208) (width 0.2) (layer "F.Cu") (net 1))
 (segment (start 147.28542 98.835) (end 146.975 98.835) (width 0.2) (layer "F.Cu") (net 1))
 (segment (start 146.975 98.835) (end 145.985 98.835) (width 0.2) (layer "F.Cu") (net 1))
 (segment (start 148.66 97.44) (end 147.265 98.835) (width 0.2) (layer "F.Cu") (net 1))
 (segment (start 147.265 98.835) (end 146.975 98.835) (width 0.2) (layer "F.Cu") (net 1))
 (segment (start 148.133 92.208) (end 148.66 92.735) (width 0.2) (layer "F.Cu") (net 1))
 (segment (start 149.83542 101.385) (end 147.28542 98.835) (width 0.2) (layer "F.Cu") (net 1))
 (segment (start 142.35 92.5) (end 142.642 92.208) (width 0.2) (layer "F.Cu") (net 1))
 (segment (start 151.575 101.385) (end 149.83542 101.385) (width 0.2) (layer "F.Cu") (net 1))
 (segment (start 154.075 101.375) (end 151.585 101.375) (width 0.2) (layer "F.Cu") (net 1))
 (segment (start 148.66 92.735) (end 148.66 97.44) (width 0.2) (layer "F.Cu") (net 1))
 (segment (start 158.415 92.735) (end 158.65 92.5) (width 0.2) (layer "F.Cu") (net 1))
 (segment (start 151.55 92.735) (end 158.415 92.735) (width 0.2) (layer "F.Cu") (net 1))
 (segment (start 148.66 92.735) (end 151.55 92.735) (width 0.2) (layer "F.Cu") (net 1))
 (segment (start 145.985 98.835) (end 145.975 98.825) (width 0.2) (layer "F.Cu") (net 1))
 (segment (start 151.585 101.375) (end 151.575 101.385) (width 0.2) (layer "F.Cu") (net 1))
 (segment (start 151.875 95.275) (end 151.55 95.275) (width 0.2) (layer "F.Cu") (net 2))
 (segment (start 154.075 100.415) (end 154.075 98.575) (width 0.2) (layer "F.Cu") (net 2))
 (segment (start 154.075 97.475) (end 151.875 95.275) (width 0.2) (layer "F.Cu") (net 2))
 (segment (start 154.075 98.575) (end 154.075 97.475) (width 0.2) (layer "F.Cu") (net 2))
 (segment (start 146.6 97.5) (end 146.975 97.875) (width 0.2) (layer "F.Cu") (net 4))
 (segment (start 146.965 97.865) (end 146.975 97.875) (width 0.2) (layer "F.Cu") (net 4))
 (segment (start 145.975 97.865) (end 146.965 97.865) (width 0.2) (layer "F.Cu") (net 4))
 (segment (start 146.6 96.545) (end 146.6 97.5) (width 0.2) (layer "F.Cu") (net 4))
 (via (at 146.6 97.375) (size 0.5) (drill 0.2) (layers "F.Cu" "B.Cu") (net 4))
 (segment (start 146.6 97.375) (end 146.6 98.5) (width 0.2) (layer "B.Cu") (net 4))
 (segment (start 146.6 98.5) (end 158.6 98.5) (width 0.2) (layer "B.Cu") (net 4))
 (segment (start 142.4 98.5) (end 146.6 98.5) (width 0.2) (layer "B.Cu") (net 4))
 (segment (start 156.625 94.5) (end 155.825 93.7) (width 0.2) (layer "F.Cu") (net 5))
 (segment (start 158.65 94.5) (end 156.625 94.5) (width 0.2) (layer "F.Cu") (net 5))
 (segment (start 144.425 94.5) (end 142.35 94.5) (width 0.2) (layer "F.Cu") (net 5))
 (segment (start 145.1 93.525) (end 145.2 93.425) (width 0.2) (layer "F.Cu") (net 5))
 (segment (start 145.2 93.425) (end 145.5 93.425) (width 0.2) (layer "F.Cu") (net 5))
 (segment (start 146.6 92.735) (end 146.19 92.735) (width 0.2) (layer "F.Cu") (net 5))
 (segment (start 145.5 93.425) (end 144.425 94.5) (width 0.2) (layer "F.Cu") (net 5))
 (segment (start 146.19 92.735) (end 145.5 93.425) (width 0.2) (layer "F.Cu") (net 5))
 (via (at 155.825 93.7) (size 0.5) (drill 0.2) (layers "F.Cu" "B.Cu") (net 5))
 (via (at 145.1 93.525) (size 0.5) (drill 0.2) (layers "F.Cu" "B.Cu") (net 5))
 (segment (start 145.275 93.7) (end 145.1 93.525) (width 0.2) (layer "B.Cu") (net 5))
 (segment (start 155.825 93.7) (end 145.275 93.7) (width 0.2) (layer "B.Cu") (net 5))
 (segment (start 145.625001 94.005) (end 145.3 94.330001) (width 0.2) (layer "F.Cu") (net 7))
 (segment (start 145.3 96.85) (end 144.8125 97.3375) (width 0.2) (layer "F.Cu") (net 7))
 (segment (start 143.65 98.5) (end 142.35 98.5) (width 0.2) (layer "F.Cu") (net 7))
 (segment (start 144.8125 97.3375) (end 143.65 98.5) (width 0.2) (layer "F.Cu") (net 7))
 (segment (start 158.65 98.5) (end 156.825 98.5) (width 0.2) (layer "F.Cu") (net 7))
 (segment (start 146.6 94.005) (end 145.625001 94.005) (width 0.2) (layer "F.Cu") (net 7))
 (segment (start 156.825 98.5) (end 155.825 97.5) (width 0.2) (layer "F.Cu") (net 7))
 (segment (start 145.3 94.330001) (end 145.3 96.85) (width 0.2) (layer "F.Cu") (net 7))
 (via (at 144.8125 97.3375) (size 0.5) (drill 0.2) (layers "F.Cu" "B.Cu") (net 7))
 (via (at 155.825 97.5) (size 0.5) (drill 0.2) (layers "F.Cu" "B.Cu") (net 7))
 (segment (start 155.223 96.898) (end 145.252 96.898) (width 0.2) (layer "B.Cu") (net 7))
 (segment (start 145.252 96.898) (end 144.8125 97.3375) (width 0.2) (layer "B.Cu") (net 7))
 (segment (start 155.825 97.5) (end 155.223 96.898) (width 0.2) (layer "B.Cu") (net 7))
 (segment (start 150.575001 94.005) (end 150.275 94.305001) (width 0.2) (layer "F.Cu") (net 8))
 (segment (start 149.725 94.85) (end 149.725 100.6) (width 0.2) (layer "F.Cu") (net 8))
 (segment (start 150.275 94.305001) (end 150.269999 94.305001) (width 0.2) (layer "F.Cu") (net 8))
 (segment (start 151.55 94.005) (end 150.575001 94.005) (width 0.2) (layer "F.Cu") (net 8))
 (segment (start 150.269999 94.305001) (end 149.725 94.85) (width 0.2) (layer "F.Cu") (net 8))
 (segment (start 149.725 101.925) (end 145.35 101.925) (width 0.2) (layer "F.Cu") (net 8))
 (segment (start 145.35 101.925) (end 143.925 100.5) (width 0.2) (layer "F.Cu") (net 8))
 (segment (start 149.725 101.925) (end 155.25 101.925) (width 0.2) (layer "F.Cu") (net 8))
 (segment (start 143.925 100.5) (end 142.35 100.5) (width 0.2) (layer "F.Cu") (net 8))
 (segment (start 156.675 100.5) (end 158.65 100.5) (width 0.2) (layer "F.Cu") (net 8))
 (segment (start 155.25 101.925) (end 156.675 100.5) (width 0.2) (layer "F.Cu") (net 8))
 (via (at 149.725 100.6) (size 0.5) (drill 0.2) (layers "F.Cu" "B.Cu") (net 8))
 (via (at 149.725 101.925) (size 0.5) (drill 0.2) (layers "F.Cu" "B.Cu") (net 8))
 (segment (start 149.725 101.925) (end 149.725 100.6) (width 0.2) (layer "B.Cu") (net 8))
 (segment (start 145.175 99.325) (end 155.675 99.325) (width 0.2) (layer "B.Cu") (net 12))
 (segment (start 156.85 100.5) (end 158.5 100.5) (width 0.2) (layer "B.Cu") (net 12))
 (segment (start 155.675 99.325) (end 156.85 100.5) (width 0.2) (layer "B.Cu") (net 12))
 (segment (start 144 100.5) (end 145.175 99.325) (width 0.2) (layer "B.Cu") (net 12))
 (segment (start 142.3 100.5) (end 144 100.5) (width 0.2) (layer "B.Cu") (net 12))
 (segment (start 154.5875 95.4125) (end 155.675 96.5) (width 0.2) (layer "F.Cu") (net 6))
 (segment (start 155.675 96.5) (end 158.65 96.5) (width 0.2) (layer "F.Cu") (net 6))
 (segment (start 144.8 95.525) (end 143.825 96.5) (width 0.2) (layer "F.Cu") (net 6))
 (segment (start 143.825 96.5) (end 142.35 96.5) (width 0.2) (layer "F.Cu") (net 6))
 (via (at 144.8 95.525) (size 0.5) (drill 0.2) (layers "F.Cu" "B.Cu") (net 6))
 (via (at 154.5875 95.4125) (size 0.5) (drill 0.2) (layers "F.Cu" "B.Cu") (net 6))
 (segment (start 144.8 95.525) (end 144.85 95.475) (width 0.2) (layer "B.Cu") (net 6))
 (segment (start 154.525 95.475) (end 154.5875 95.4125) (width 0.2) (layer "B.Cu") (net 6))
 (segment (start 144.85 95.475) (end 154.525 95.475) (width 0.2) (layer "B.Cu") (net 6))
 (segment (start 142.4 92.5) (end 158.6 92.5) (width 0.2) (layer "B.Cu") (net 9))
 (segment (start 142.1 94.5) (end 158.65 94.5) (width 0.2) (layer "B.Cu") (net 10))
 (segment (start 142.6 96.5) (end 158.65 96.5) (width 0.2) (layer "B.Cu") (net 11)))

